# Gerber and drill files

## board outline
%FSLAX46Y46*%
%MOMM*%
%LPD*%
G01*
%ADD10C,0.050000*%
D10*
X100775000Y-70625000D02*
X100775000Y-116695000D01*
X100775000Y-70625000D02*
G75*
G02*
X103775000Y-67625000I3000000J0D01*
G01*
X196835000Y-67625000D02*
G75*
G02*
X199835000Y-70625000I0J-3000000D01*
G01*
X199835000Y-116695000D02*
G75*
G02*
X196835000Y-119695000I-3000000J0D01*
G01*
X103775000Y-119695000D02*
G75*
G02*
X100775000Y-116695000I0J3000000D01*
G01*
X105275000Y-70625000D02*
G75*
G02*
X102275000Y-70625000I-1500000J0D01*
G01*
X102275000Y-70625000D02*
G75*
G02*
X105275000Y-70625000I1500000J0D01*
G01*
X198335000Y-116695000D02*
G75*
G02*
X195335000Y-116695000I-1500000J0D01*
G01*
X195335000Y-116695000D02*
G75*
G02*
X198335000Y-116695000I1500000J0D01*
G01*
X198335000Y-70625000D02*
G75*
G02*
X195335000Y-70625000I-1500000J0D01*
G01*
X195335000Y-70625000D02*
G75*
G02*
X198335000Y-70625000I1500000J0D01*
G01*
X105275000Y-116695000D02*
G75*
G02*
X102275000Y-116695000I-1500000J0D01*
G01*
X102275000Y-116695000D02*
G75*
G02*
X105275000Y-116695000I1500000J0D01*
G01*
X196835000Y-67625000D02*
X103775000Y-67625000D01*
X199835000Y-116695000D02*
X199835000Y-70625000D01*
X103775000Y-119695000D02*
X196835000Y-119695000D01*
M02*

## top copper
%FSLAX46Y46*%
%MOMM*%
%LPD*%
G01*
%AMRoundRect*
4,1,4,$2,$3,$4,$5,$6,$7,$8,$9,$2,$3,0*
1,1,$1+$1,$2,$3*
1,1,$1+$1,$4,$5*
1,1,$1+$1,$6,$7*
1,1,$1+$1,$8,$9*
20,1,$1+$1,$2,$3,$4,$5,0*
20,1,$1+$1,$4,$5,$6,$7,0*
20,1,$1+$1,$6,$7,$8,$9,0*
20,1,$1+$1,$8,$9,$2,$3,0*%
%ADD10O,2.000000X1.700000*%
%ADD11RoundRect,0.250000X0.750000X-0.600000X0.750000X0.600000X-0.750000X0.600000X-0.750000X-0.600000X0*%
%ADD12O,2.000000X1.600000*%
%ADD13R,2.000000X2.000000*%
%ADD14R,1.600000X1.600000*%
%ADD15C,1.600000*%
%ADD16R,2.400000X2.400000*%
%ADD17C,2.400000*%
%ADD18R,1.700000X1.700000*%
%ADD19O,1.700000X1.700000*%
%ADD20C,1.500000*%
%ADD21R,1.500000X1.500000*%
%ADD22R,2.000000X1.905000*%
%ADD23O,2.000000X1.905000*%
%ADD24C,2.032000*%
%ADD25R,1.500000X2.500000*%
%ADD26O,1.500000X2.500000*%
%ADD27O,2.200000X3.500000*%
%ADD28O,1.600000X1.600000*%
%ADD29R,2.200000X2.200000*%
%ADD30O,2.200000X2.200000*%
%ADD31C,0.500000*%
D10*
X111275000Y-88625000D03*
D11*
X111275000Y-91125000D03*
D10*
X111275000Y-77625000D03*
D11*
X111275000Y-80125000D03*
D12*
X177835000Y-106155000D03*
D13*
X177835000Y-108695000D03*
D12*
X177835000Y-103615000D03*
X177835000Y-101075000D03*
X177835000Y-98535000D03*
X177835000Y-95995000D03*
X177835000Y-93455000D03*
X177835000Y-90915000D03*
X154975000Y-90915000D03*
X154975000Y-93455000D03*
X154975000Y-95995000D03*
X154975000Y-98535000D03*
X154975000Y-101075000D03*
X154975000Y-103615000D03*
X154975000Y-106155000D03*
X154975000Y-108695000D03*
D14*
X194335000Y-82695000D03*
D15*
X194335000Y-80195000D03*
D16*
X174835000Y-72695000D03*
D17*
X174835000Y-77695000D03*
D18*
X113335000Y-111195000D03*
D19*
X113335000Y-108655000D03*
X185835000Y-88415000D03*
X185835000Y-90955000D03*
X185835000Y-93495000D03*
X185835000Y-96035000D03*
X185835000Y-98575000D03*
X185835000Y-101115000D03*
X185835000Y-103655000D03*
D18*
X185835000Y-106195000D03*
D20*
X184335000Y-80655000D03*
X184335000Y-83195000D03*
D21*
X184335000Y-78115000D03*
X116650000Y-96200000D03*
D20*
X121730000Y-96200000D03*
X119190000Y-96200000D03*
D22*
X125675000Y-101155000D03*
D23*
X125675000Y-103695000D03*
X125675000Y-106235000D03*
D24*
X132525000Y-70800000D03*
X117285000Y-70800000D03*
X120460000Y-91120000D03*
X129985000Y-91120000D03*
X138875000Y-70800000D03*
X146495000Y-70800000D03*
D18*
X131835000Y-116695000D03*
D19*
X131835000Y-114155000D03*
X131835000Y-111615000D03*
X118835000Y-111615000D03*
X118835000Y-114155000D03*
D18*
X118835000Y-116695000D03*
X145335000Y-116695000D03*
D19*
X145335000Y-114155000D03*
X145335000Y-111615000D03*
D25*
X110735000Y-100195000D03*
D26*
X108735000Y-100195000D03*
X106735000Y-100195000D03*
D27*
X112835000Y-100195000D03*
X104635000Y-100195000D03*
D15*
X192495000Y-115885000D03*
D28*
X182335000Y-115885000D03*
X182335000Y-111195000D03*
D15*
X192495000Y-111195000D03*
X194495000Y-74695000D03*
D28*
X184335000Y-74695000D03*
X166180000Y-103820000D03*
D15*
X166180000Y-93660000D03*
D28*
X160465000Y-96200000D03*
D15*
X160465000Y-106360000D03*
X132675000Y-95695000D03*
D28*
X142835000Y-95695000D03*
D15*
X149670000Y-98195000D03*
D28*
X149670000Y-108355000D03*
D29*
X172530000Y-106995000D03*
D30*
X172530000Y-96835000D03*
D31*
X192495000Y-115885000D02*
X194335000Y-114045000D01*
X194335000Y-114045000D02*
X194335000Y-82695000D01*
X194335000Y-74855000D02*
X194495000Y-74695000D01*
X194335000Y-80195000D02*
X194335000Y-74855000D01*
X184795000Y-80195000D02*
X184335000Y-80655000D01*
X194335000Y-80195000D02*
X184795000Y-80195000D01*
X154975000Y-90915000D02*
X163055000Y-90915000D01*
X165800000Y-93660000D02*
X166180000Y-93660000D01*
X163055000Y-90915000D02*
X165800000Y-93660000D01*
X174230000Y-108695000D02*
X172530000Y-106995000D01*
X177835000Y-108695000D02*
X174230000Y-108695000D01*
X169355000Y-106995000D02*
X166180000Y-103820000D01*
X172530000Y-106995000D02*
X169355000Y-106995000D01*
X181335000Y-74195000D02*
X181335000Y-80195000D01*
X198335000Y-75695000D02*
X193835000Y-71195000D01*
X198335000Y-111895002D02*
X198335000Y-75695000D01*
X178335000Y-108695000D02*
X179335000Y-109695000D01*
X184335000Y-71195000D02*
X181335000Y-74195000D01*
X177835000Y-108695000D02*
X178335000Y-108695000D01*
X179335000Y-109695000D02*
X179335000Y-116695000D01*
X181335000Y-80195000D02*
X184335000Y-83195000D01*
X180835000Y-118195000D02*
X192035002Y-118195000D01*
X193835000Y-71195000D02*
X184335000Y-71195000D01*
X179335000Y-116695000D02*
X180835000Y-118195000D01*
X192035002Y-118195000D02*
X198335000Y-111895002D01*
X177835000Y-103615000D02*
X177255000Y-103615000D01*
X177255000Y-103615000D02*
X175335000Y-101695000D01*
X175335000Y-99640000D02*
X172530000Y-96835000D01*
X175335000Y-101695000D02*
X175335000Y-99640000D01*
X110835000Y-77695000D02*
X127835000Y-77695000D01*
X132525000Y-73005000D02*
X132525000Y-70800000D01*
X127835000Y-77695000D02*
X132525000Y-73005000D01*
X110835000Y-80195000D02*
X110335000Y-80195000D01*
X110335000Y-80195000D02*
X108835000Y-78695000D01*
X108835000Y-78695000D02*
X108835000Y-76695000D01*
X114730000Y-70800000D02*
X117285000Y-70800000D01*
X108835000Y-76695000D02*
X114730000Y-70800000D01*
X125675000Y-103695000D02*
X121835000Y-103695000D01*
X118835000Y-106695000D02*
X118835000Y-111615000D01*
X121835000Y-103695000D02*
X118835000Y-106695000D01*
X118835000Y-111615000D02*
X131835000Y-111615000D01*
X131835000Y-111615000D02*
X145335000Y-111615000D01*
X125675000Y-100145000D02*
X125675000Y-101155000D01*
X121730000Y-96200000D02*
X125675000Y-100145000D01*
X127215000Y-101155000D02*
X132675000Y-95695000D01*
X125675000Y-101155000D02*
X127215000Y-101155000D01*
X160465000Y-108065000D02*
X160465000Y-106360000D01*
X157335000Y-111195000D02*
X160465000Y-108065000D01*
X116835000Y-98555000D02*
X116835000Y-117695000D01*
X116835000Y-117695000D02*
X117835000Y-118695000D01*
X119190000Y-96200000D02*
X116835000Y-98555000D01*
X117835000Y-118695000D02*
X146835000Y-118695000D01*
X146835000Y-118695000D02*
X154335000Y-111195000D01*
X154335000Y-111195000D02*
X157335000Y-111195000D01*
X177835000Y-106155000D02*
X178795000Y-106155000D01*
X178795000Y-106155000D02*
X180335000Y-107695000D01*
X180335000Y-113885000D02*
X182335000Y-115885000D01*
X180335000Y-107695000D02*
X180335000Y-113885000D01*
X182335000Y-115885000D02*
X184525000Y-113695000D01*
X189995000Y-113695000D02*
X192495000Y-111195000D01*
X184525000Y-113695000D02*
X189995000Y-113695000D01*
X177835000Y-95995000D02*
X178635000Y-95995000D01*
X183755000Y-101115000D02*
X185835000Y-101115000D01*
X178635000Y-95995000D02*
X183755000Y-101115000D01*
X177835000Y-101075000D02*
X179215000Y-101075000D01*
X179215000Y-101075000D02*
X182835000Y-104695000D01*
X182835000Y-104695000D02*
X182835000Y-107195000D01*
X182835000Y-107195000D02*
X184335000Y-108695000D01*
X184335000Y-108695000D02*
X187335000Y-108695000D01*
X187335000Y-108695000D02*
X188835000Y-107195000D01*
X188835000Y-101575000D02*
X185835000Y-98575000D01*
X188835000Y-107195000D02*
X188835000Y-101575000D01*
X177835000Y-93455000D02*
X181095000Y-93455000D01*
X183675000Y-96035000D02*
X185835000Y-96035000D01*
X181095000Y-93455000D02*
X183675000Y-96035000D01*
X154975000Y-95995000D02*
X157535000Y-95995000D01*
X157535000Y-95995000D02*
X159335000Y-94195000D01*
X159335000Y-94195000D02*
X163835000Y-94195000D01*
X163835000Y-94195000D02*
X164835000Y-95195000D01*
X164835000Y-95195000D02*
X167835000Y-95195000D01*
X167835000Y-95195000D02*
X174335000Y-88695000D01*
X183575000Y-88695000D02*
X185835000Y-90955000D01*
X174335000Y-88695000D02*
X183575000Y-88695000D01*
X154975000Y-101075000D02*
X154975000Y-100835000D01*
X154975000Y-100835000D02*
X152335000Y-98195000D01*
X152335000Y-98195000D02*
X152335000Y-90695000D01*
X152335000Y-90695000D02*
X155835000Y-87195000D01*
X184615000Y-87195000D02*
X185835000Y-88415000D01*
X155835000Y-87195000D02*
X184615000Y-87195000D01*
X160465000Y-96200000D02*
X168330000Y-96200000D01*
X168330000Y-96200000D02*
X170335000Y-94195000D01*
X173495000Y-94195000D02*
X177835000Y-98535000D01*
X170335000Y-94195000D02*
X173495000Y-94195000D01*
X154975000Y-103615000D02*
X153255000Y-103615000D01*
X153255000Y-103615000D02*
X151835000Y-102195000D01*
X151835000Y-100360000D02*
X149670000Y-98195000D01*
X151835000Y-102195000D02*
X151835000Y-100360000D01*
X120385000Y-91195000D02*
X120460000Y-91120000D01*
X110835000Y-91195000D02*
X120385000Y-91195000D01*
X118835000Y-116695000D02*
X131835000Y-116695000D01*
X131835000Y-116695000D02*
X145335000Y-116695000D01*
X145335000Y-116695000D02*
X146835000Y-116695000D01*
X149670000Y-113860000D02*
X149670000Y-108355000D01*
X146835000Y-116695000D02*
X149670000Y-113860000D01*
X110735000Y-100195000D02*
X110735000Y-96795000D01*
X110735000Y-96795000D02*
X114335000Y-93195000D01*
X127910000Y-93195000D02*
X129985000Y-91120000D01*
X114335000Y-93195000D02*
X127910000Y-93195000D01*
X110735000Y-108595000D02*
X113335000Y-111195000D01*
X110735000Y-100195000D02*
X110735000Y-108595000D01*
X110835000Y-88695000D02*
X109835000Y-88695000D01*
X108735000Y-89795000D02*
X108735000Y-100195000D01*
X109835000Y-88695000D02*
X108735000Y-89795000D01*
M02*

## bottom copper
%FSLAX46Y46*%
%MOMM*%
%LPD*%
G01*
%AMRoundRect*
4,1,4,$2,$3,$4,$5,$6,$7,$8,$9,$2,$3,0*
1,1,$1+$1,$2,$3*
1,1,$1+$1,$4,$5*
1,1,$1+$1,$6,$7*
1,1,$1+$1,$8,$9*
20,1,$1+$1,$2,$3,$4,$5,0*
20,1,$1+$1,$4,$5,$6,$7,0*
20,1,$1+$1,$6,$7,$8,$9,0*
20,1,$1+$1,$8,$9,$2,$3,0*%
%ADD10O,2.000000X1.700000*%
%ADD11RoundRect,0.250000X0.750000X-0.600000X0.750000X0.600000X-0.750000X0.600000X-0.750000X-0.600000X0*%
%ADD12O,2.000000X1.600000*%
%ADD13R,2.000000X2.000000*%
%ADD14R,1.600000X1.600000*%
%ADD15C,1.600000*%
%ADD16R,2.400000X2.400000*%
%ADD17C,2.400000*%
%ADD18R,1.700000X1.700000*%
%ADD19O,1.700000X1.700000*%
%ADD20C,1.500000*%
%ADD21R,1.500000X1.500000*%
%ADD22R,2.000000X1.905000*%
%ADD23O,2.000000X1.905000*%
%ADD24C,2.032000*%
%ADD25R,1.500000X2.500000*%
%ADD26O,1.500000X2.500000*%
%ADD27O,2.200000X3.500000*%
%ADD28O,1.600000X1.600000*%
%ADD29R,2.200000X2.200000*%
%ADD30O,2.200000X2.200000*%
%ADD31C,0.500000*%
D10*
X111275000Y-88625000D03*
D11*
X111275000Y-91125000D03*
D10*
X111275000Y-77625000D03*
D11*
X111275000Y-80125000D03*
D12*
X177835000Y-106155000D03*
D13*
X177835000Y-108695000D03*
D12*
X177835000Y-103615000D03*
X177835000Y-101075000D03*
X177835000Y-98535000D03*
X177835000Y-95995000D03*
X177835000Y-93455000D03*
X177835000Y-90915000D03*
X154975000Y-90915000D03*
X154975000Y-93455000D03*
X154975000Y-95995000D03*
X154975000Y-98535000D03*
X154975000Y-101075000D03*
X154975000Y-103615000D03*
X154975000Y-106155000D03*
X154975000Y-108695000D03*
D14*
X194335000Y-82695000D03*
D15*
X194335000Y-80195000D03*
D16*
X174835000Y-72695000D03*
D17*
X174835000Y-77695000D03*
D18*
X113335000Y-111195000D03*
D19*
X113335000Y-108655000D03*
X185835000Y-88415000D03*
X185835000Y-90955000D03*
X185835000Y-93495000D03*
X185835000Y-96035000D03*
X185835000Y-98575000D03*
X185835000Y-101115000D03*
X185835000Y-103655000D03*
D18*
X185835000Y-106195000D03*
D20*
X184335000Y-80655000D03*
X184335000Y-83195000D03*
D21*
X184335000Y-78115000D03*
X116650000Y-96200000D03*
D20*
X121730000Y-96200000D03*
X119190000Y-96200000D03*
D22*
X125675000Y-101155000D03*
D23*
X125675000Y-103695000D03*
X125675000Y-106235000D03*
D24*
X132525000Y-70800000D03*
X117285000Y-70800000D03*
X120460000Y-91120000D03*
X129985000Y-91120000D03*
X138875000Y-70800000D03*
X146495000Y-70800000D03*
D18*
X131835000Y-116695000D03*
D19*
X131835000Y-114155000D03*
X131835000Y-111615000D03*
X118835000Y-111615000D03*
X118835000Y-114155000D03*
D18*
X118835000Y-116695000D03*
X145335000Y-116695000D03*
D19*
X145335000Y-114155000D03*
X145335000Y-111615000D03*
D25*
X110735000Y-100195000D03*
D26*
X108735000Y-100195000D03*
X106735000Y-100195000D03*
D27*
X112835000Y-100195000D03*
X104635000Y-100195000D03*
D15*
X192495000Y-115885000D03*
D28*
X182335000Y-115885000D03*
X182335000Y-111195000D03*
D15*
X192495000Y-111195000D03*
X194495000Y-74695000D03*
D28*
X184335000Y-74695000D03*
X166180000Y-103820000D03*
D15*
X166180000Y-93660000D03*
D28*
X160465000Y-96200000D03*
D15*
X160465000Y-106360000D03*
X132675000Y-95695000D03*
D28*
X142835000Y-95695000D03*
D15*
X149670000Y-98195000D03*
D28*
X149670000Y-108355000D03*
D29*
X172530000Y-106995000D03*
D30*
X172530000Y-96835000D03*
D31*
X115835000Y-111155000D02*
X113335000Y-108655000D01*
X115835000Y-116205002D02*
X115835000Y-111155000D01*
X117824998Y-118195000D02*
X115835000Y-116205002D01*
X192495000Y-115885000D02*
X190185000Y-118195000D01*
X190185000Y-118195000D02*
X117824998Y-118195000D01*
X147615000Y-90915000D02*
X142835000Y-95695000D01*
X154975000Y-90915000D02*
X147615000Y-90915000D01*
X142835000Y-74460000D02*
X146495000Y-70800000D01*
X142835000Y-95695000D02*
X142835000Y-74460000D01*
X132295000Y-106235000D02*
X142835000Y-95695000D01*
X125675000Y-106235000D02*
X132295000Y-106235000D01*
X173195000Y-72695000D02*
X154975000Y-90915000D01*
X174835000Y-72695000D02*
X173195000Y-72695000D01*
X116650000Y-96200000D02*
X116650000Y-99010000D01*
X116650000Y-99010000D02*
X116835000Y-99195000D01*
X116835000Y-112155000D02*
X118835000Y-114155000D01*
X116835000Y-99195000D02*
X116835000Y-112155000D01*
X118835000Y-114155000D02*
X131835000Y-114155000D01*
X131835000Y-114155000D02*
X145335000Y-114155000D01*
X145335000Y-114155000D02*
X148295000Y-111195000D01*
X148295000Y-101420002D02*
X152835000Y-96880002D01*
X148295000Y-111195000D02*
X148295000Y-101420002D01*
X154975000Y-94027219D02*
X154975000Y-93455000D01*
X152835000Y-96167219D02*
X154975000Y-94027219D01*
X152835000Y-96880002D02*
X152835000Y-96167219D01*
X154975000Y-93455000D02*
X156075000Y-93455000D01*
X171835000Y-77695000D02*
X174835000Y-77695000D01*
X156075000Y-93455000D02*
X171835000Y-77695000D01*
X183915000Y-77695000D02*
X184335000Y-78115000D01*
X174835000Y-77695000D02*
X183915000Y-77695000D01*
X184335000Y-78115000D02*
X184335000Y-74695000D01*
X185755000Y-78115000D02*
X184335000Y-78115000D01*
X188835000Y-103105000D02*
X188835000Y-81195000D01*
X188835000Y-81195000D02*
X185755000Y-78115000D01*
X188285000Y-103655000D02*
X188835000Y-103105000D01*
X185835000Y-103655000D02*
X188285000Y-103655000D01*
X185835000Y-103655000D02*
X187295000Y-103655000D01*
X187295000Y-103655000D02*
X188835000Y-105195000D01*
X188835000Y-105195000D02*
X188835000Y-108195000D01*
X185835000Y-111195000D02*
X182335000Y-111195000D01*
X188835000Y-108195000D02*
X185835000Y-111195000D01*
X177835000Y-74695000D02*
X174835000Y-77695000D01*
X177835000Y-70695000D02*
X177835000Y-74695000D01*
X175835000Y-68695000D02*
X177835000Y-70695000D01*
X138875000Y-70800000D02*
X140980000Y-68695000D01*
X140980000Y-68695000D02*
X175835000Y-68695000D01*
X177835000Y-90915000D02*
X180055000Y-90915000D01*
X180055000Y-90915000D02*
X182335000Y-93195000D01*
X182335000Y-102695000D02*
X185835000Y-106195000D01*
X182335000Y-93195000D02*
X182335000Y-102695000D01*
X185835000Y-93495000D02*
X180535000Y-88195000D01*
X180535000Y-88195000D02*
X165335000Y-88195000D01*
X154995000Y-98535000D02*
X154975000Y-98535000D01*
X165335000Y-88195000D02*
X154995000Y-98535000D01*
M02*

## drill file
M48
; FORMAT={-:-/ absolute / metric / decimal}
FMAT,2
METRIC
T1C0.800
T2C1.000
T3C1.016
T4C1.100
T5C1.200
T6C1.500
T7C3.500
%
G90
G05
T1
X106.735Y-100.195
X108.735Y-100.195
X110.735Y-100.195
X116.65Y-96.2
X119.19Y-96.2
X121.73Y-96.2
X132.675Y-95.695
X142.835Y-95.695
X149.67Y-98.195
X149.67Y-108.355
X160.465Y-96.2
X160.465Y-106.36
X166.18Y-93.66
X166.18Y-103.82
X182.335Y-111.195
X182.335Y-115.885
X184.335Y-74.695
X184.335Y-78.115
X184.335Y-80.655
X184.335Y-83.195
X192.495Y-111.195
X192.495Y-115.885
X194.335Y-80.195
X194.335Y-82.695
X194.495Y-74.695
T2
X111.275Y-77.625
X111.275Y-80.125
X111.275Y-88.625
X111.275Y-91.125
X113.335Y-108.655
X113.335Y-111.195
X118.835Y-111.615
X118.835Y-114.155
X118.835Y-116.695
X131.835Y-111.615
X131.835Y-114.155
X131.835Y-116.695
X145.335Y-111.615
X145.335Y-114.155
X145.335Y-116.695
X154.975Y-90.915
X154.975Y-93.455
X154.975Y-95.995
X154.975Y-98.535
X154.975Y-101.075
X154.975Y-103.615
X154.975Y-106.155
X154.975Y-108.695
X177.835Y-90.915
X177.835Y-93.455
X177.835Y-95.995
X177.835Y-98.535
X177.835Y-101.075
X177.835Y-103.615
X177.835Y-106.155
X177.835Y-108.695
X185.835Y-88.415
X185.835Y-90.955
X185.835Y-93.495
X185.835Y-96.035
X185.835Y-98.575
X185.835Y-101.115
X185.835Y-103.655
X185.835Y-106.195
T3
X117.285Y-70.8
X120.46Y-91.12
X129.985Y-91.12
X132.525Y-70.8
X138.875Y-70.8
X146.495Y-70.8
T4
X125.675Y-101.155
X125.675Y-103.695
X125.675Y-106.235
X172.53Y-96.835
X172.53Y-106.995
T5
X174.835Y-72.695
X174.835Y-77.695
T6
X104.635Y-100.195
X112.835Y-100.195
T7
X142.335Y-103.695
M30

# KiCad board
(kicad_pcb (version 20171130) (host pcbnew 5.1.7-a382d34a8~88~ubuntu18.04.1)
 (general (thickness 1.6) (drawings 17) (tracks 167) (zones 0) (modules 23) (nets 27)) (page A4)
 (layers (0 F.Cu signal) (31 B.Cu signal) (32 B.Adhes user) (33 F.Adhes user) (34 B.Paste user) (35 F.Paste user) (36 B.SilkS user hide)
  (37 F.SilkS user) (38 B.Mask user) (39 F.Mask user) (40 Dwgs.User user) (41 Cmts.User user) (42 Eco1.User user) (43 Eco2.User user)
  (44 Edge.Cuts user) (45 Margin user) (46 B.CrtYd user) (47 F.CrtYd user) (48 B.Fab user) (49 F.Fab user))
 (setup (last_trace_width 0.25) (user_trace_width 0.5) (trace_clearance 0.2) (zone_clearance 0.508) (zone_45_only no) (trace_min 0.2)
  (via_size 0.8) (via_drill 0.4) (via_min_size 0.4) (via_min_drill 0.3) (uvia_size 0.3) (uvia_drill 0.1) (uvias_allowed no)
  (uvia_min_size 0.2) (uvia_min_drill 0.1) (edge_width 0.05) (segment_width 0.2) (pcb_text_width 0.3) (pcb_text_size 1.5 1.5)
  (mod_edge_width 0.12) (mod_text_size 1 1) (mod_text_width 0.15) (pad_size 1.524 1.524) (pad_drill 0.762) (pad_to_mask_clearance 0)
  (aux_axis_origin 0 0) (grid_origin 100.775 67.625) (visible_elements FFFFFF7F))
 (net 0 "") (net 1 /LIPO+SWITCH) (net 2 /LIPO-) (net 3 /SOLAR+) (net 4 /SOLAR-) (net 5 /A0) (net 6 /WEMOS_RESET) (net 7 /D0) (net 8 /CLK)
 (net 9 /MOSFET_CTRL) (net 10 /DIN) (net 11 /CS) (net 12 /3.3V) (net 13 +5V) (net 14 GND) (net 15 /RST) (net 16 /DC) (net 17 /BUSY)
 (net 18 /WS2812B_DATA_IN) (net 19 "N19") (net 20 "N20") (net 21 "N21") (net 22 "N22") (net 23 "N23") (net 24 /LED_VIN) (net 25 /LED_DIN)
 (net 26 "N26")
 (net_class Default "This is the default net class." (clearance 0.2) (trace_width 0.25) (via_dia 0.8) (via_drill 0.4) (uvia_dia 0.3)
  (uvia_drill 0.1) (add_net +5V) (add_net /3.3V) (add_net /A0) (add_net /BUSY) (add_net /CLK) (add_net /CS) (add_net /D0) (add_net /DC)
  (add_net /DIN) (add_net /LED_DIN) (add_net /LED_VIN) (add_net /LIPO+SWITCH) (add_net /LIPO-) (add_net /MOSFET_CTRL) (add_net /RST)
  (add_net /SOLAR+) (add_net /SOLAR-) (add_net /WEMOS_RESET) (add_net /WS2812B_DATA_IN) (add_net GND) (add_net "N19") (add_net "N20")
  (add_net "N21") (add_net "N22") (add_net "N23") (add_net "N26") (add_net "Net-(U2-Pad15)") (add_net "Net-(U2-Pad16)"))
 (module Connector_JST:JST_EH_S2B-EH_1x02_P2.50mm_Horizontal (layer F.Cu) (at 111.275 91.125 90)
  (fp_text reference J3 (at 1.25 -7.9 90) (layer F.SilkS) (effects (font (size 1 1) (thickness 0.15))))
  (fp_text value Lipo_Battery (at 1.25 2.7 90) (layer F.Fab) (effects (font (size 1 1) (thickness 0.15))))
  (pad 2 thru_hole oval (at 2.5 0 90) (size 1.7 2) (drill 1) (layers *.Cu *.Mask) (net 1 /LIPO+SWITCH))
  (pad 1 thru_hole roundrect (at 0 0 90) (size 1.7 2) (drill 1) (layers *.Cu *.Mask) (roundrect_rratio 0.147059) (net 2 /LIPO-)))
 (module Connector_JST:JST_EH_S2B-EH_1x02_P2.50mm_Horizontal (layer F.Cu) (at 111.275 80.125 90)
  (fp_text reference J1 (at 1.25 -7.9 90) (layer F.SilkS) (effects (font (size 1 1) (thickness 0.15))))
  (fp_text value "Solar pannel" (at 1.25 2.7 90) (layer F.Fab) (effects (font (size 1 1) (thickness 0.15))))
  (pad 2 thru_hole oval (at 2.5 0 90) (size 1.7 2) (drill 1) (layers *.Cu *.Mask) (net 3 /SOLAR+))
  (pad 1 thru_hole roundrect (at 0 0 90) (size 1.7 2) (drill 1) (layers *.Cu *.Mask) (roundrect_rratio 0.147059) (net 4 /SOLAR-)))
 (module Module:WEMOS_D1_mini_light (layer F.Cu) (at 177.835 108.695 180)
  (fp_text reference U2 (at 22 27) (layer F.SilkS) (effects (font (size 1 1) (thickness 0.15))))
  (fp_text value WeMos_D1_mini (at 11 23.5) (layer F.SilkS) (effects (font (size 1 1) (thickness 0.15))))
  (pad 2 thru_hole oval (at 0 2.54 180) (size 2 1.6) (drill 1) (layers *.Cu *.Mask) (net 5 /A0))
  (pad 1 thru_hole rect (at 0 0 180) (size 2 2) (drill 1) (layers *.Cu *.Mask) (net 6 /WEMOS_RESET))
  (pad 3 thru_hole oval (at 0 5.08 180) (size 2 1.6) (drill 1) (layers *.Cu *.Mask) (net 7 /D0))
  (pad 4 thru_hole oval (at 0 7.62 180) (size 2 1.6) (drill 1) (layers *.Cu *.Mask) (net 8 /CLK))
  (pad 5 thru_hole oval (at 0 10.16 180) (size 2 1.6) (drill 1) (layers *.Cu *.Mask) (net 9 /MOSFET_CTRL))
  (pad 6 thru_hole oval (at 0 12.7 180) (size 2 1.6) (drill 1) (layers *.Cu *.Mask) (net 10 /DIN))
  (pad 7 thru_hole oval (at 0 15.24 180) (size 2 1.6) (drill 1) (layers *.Cu *.Mask) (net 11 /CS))
  (pad 8 thru_hole oval (at 0 17.78 180) (size 2 1.6) (drill 1) (layers *.Cu *.Mask) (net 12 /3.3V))
  (pad 9 thru_hole oval (at 22.86 17.78 180) (size 2 1.6) (drill 1) (layers *.Cu *.Mask) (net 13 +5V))
  (pad 10 thru_hole oval (at 22.86 15.24 180) (size 2 1.6) (drill 1) (layers *.Cu *.Mask) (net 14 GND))
  (pad 11 thru_hole oval (at 22.86 12.7 180) (size 2 1.6) (drill 1) (layers *.Cu *.Mask) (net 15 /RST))
  (pad 12 thru_hole oval (at 22.86 10.16 180) (size 2 1.6) (drill 1) (layers *.Cu *.Mask) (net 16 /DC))
  (pad 13 thru_hole oval (at 22.86 7.62 180) (size 2 1.6) (drill 1) (layers *.Cu *.Mask) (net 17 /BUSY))
  (pad 14 thru_hole oval (at 22.86 5.08 180) (size 2 1.6) (drill 1) (layers *.Cu *.Mask) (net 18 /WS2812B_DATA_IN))
  (pad 15 thru_hole oval (at 22.86 2.54 180) (size 2 1.6) (drill 1) (layers *.Cu *.Mask))
  (pad 16 thru_hole oval (at 22.86 0 180) (size 2 1.6) (drill 1) (layers *.Cu *.Mask)))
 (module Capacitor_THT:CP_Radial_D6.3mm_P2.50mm (layer F.Cu) (at 194.335 82.695 90)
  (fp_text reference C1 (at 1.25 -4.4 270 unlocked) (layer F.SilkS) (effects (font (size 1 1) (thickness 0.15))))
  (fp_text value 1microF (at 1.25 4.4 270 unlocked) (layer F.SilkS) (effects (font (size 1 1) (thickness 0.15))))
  (pad 1 thru_hole rect (at 0 0 90) (size 1.6 1.6) (drill 0.8) (layers *.Cu *.Mask) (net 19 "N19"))
  (pad 2 thru_hole circle (at 2.5 0 90) (size 1.6 1.6) (drill 0.8) (layers *.Cu *.Mask) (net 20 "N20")))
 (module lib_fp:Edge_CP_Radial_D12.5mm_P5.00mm (layer F.Cu) (at 174.835 75.195 270)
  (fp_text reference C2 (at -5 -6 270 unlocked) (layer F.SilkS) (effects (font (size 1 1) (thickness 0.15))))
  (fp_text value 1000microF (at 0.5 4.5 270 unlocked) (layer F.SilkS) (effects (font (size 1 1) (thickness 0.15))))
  (pad 1 thru_hole rect (at -2.5 0 270) (size 2.4 2.4) (drill 1.2) (layers *.Cu *.Mask) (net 13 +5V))
  (pad 2 thru_hole circle (at 2.5 0 270) (size 2.4 2.4) (drill 1.2) (layers *.Cu *.Mask) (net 14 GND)))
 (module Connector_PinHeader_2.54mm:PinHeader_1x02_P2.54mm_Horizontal (layer F.Cu) (at 113.335 111.195 180)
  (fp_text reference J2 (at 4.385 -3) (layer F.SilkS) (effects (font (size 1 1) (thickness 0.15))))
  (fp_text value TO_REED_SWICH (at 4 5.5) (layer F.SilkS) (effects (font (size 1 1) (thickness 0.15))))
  (pad 1 thru_hole rect (at 0 0 180) (size 1.7 1.7) (drill 1) (layers *.Cu *.Mask) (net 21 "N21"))
  (pad 2 thru_hole oval (at 0 2.54 180) (size 1.7 1.7) (drill 1) (layers *.Cu *.Mask) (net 19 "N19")))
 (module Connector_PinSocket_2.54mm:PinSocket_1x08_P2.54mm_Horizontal (layer F.Cu) (at 185.835 106.195 180)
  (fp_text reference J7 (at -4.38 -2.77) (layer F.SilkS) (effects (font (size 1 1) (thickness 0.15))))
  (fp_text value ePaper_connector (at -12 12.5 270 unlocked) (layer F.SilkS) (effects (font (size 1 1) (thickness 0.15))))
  (pad 8 thru_hole oval (at 0 17.78 180) (size 1.7 1.7) (drill 1) (layers *.Cu *.Mask) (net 17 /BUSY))
  (pad 7 thru_hole oval (at 0 15.24 180) (size 1.7 1.7) (drill 1) (layers *.Cu *.Mask) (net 15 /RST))
  (pad 6 thru_hole oval (at 0 12.7 180) (size 1.7 1.7) (drill 1) (layers *.Cu *.Mask) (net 16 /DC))
  (pad 5 thru_hole oval (at 0 10.16 180) (size 1.7 1.7) (drill 1) (layers *.Cu *.Mask) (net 11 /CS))
  (pad 4 thru_hole oval (at 0 7.62 180) (size 1.7 1.7) (drill 1) (layers *.Cu *.Mask) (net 8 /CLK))
  (pad 3 thru_hole oval (at 0 5.08 180) (size 1.7 1.7) (drill 1) (layers *.Cu *.Mask) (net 10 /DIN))
  (pad 2 thru_hole oval (at 0 2.54 180) (size 1.7 1.7) (drill 1) (layers *.Cu *.Mask) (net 14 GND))
  (pad 1 thru_hole rect (at 0 0 180) (size 1.7 1.7) (drill 1) (layers *.Cu *.Mask) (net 12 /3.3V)))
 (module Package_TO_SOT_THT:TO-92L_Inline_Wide (layer F.Cu) (at 184.335 78.115 270)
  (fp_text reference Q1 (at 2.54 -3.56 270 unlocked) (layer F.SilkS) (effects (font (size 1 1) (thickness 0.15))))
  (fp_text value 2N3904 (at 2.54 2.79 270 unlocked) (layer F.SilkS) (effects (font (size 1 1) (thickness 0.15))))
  (pad 2 thru_hole circle (at 2.54 0 270) (size 1.5 1.5) (drill 0.8) (layers *.Cu *.Mask) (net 20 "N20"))
  (pad 3 thru_hole circle (at 5.08 0 270) (size 1.5 1.5) (drill 0.8) (layers *.Cu *.Mask) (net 14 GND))
  (pad 1 thru_hole rect (at 0 0 270) (size 1.5 1.5) (drill 0.8) (layers *.Cu *.Mask) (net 6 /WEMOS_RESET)))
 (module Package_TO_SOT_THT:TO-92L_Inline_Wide (layer F.Cu) (at 116.65 96.2)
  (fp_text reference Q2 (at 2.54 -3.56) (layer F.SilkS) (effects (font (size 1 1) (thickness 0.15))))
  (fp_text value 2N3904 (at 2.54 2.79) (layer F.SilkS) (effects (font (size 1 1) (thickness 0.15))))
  (pad 1 thru_hole rect (at 0 0) (size 1.5 1.5) (drill 0.8) (layers *.Cu *.Mask) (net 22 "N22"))
  (pad 3 thru_hole circle (at 5.08 0) (size 1.5 1.5) (drill 0.8) (layers *.Cu *.Mask) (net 14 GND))
  (pad 2 thru_hole circle (at 2.54 0) (size 1.5 1.5) (drill 0.8) (layers *.Cu *.Mask) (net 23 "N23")))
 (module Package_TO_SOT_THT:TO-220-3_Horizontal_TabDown (layer F.Cu) (at 125.675 101.155 270)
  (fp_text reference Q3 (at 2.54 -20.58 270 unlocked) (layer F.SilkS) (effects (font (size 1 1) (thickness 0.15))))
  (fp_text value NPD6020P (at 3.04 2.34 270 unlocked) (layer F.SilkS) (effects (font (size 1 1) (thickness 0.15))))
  (pad "" np_thru_hole oval (at 2.54 -16.66 270) (size 3.5 3.5) (drill 3.5) (layers *.Cu *.Mask))
  (pad 1 thru_hole rect (at 0 0 270) (size 1.905 2) (drill 1.1) (layers *.Cu *.Mask) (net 22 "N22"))
  (pad 2 thru_hole oval (at 2.54 0 270) (size 1.905 2) (drill 1.1) (layers *.Cu *.Mask) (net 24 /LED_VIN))
  (pad 3 thru_hole oval (at 5.08 0 270) (size 1.905 2) (drill 1.1) (layers *.Cu *.Mask) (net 13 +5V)))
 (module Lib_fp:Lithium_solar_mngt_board (layer F.Cu) (at 135.065 66.99)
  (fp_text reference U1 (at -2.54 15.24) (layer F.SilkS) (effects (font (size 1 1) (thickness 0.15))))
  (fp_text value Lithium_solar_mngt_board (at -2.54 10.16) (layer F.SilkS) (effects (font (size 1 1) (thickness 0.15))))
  (pad 1 thru_hole circle (at -2.54 3.81) (size 2.032 2.032) (drill 1.016) (layers *.Cu *.Mask) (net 3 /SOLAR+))
  (pad 2 thru_hole circle (at -17.78 3.81) (size 2.032 2.032) (drill 1.016) (layers *.Cu *.Mask) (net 4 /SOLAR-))
  (pad 4 thru_hole circle (at -14.605 24.13) (size 2.032 2.032) (drill 1.016) (layers *.Cu *.Mask) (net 2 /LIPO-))
  (pad 3 thru_hole circle (at -5.08 24.13) (size 2.032 2.032) (drill 1.016) (layers *.Cu *.Mask) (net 21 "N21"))
  (pad 6 thru_hole circle (at 3.81 3.81) (size 2.032 2.032) (drill 1.016) (layers *.Cu *.Mask) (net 14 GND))
  (pad 5 thru_hole circle (at 11.43 3.81) (size 2.032 2.032) (drill 1.016) (layers *.Cu *.Mask) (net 13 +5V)))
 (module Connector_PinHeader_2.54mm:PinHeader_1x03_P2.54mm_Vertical (layer F.Cu) (at 131.835 116.695 180)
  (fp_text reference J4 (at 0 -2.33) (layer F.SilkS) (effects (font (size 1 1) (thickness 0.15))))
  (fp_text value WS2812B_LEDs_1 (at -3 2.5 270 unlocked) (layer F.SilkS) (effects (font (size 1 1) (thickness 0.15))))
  (pad 1 thru_hole rect (at 0 0 180) (size 1.7 1.7) (drill 1) (layers *.Cu *.Mask) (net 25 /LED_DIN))
  (pad 2 thru_hole oval (at 0 2.54 180) (size 1.7 1.7) (drill 1) (layers *.Cu *.Mask) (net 14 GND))
  (pad 3 thru_hole oval (at 0 5.08 180) (size 1.7 1.7) (drill 1) (layers *.Cu *.Mask) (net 24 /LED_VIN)))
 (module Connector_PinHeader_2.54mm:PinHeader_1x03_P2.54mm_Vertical (layer F.Cu) (at 118.835 116.695 180)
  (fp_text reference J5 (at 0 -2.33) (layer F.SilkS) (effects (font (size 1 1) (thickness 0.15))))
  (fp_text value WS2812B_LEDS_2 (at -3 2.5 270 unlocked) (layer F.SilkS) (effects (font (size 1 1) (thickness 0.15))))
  (pad 3 thru_hole oval (at 0 5.08 180) (size 1.7 1.7) (drill 1) (layers *.Cu *.Mask) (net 24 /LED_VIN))
  (pad 2 thru_hole oval (at 0 2.54 180) (size 1.7 1.7) (drill 1) (layers *.Cu *.Mask) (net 14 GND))
  (pad 1 thru_hole rect (at 0 0 180) (size 1.7 1.7) (drill 1) (layers *.Cu *.Mask) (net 25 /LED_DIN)))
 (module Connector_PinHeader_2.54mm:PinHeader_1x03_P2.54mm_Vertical (layer F.Cu) (at 145.335 116.695 180)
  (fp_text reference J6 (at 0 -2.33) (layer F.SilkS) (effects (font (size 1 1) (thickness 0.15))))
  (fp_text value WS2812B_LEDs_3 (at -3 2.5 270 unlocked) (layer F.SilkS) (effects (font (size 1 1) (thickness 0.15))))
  (pad 1 thru_hole rect (at 0 0 180) (size 1.7 1.7) (drill 1) (layers *.Cu *.Mask) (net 25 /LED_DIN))
  (pad 2 thru_hole oval (at 0 2.54 180) (size 1.7 1.7) (drill 1) (layers *.Cu *.Mask) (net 14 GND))
  (pad 3 thru_hole oval (at 0 5.08 180) (size 1.7 1.7) (drill 1) (layers *.Cu *.Mask) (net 24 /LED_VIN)))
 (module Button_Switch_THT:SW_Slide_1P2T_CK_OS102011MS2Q (layer F.Cu) (at 110.735 100.195 180)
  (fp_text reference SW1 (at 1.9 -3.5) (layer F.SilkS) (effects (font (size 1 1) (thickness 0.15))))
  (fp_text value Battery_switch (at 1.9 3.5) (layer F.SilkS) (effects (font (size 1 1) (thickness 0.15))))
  (pad 1 thru_hole rect (at 0 0 180) (size 1.5 2.5) (drill 0.8) (layers *.Cu *.Mask) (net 21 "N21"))
  (pad 2 thru_hole oval (at 2 0 180) (size 1.5 2.5) (drill 0.8) (layers *.Cu *.Mask) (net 1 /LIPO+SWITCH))
  (pad 3 thru_hole oval (at 4 0 180) (size 1.5 2.5) (drill 0.8) (layers *.Cu *.Mask))
  (pad "" thru_hole oval (at -2.1 0 180) (size 2.2 3.5) (drill 1.5) (layers *.Cu *.Mask))
  (pad "" thru_hole oval (at 6.1 0 180) (size 2.2 3.5) (drill 1.5) (layers *.Cu *.Mask)))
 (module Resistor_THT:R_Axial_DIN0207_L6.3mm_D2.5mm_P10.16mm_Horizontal (layer F.Cu) (at 192.495 115.885 180)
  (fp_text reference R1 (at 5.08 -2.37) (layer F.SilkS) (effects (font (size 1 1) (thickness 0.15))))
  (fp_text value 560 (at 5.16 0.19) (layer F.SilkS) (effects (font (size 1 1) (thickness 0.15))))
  (pad 1 thru_hole circle (at 0 0 180) (size 1.6 1.6) (drill 0.8) (layers *.Cu *.Mask) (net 19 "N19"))
  (pad 2 thru_hole oval (at 10.16 0 180) (size 1.6 1.6) (drill 0.8) (layers *.Cu *.Mask) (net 5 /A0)))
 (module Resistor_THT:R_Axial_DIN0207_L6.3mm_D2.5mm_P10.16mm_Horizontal (layer F.Cu) (at 192.495 111.195 180)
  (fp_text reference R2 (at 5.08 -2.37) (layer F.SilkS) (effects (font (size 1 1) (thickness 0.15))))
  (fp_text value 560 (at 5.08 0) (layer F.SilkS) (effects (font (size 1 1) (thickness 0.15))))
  (pad 2 thru_hole oval (at 10.16 0 180) (size 1.6 1.6) (drill 0.8) (layers *.Cu *.Mask) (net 14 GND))
  (pad 1 thru_hole circle (at 0 0 180) (size 1.6 1.6) (drill 0.8) (layers *.Cu *.Mask) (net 5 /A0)))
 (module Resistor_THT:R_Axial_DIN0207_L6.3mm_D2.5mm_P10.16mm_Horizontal (layer F.Cu) (at 194.495 74.695 180)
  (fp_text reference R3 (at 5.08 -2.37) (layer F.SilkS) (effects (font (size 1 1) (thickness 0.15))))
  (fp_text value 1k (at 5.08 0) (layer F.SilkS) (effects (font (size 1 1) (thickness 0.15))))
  (pad 1 thru_hole circle (at 0 0 180) (size 1.6 1.6) (drill 0.8) (layers *.Cu *.Mask) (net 20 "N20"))
  (pad 2 thru_hole oval (at 10.16 0 180) (size 1.6 1.6) (drill 0.8) (layers *.Cu *.Mask) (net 14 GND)))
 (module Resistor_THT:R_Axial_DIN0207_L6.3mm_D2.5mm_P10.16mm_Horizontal (layer F.Cu) (at 166.18 93.66 270)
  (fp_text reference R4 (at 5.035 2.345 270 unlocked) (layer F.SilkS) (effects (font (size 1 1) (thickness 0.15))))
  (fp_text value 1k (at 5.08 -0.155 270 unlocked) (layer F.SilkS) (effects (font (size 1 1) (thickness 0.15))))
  (pad 2 thru_hole oval (at 10.16 0 270) (size 1.6 1.6) (drill 0.8) (layers *.Cu *.Mask) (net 6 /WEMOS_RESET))
  (pad 1 thru_hole circle (at 0 0 270) (size 1.6 1.6) (drill 0.8) (layers *.Cu *.Mask) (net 13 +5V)))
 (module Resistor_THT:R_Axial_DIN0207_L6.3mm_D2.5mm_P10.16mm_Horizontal (layer F.Cu) (at 160.465 106.36 90)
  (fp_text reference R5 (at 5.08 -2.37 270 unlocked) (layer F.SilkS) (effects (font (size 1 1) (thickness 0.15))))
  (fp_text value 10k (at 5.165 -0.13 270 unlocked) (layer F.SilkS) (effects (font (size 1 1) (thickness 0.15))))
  (pad 2 thru_hole oval (at 10.16 0 90) (size 1.6 1.6) (drill 0.8) (layers *.Cu *.Mask) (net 9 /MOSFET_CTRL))
  (pad 1 thru_hole circle (at 0 0 90) (size 1.6 1.6) (drill 0.8) (layers *.Cu *.Mask) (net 23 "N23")))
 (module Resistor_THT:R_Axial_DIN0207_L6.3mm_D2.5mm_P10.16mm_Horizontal (layer F.Cu) (at 132.675 95.695)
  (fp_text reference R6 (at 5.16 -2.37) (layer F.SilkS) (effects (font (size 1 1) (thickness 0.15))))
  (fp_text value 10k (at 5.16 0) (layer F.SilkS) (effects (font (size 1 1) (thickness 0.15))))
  (pad 1 thru_hole circle (at 0 0) (size 1.6 1.6) (drill 0.8) (layers *.Cu *.Mask) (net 22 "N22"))
  (pad 2 thru_hole oval (at 10.16 0) (size 1.6 1.6) (drill 0.8) (layers *.Cu *.Mask) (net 13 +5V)))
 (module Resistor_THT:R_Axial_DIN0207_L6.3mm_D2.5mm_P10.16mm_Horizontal (layer F.Cu) (at 149.67 98.195 270)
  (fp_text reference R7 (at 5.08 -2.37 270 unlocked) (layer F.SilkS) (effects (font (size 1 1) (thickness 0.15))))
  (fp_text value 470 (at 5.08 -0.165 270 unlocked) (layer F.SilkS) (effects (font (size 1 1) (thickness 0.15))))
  (pad 1 thru_hole circle (at 0 0 270) (size 1.6 1.6) (drill 0.8) (layers *.Cu *.Mask) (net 18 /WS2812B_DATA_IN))
  (pad 2 thru_hole oval (at 10.16 0 270) (size 1.6 1.6) (drill 0.8) (layers *.Cu *.Mask) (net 25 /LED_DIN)))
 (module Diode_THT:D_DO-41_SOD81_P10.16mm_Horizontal (layer F.Cu) (at 172.53 106.995 90)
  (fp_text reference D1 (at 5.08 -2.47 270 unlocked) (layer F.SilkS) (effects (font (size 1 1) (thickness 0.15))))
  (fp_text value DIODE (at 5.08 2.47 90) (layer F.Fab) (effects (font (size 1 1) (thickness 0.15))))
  (pad 1 thru_hole rect (at 0 0 90) (size 2.2 2.2) (drill 1.1) (layers *.Cu *.Mask) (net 6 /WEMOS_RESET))
  (pad 2 thru_hole oval (at 10.16 0 90) (size 2.2 2.2) (drill 1.1) (layers *.Cu *.Mask) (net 7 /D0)))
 (gr_line (start 100.775 70.625) (end 100.775 116.695) (layer Edge.Cuts) (width 0.05))
 (gr_arc (start 103.775 70.625) (end 103.775 67.625) (angle -90) (layer Edge.Cuts) (width 0.05))
 (gr_arc (start 196.835 70.625) (end 199.835 70.625) (angle -90) (layer Edge.Cuts) (width 0.05))
 (gr_arc (start 196.835 116.695) (end 196.835 119.695) (angle -90) (layer Edge.Cuts) (width 0.05))
 (gr_arc (start 103.775 116.695) (end 100.775 116.695) (angle -90) (layer Edge.Cuts) (width 0.05))
 (gr_circle (center 103.775 70.625) (end 102.275 70.625) (layer Edge.Cuts) (width 0.05))
 (gr_circle (center 196.835 116.695) (end 198.335 116.695) (layer Edge.Cuts) (width 0.05))
 (gr_circle (center 196.835 70.625) (end 198.335 70.625) (layer Edge.Cuts) (width 0.05))
 (gr_circle (center 103.775 116.695) (end 102.275 116.695) (layer Edge.Cuts) (width 0.05))
 (gr_line (start 196.835 67.625) (end 103.775 67.625) (layer Edge.Cuts) (width 0.05))
 (gr_line (start 199.835 116.695) (end 199.835 70.625) (layer Edge.Cuts) (width 0.05))
 (gr_line (start 103.775 119.695) (end 196.835 119.695) (layer Edge.Cuts) (width 0.05))
 (segment (start 192.495 115.885) (end 194.335 114.045) (width 0.5) (layer F.Cu) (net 19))
 (segment (start 194.335 114.045) (end 194.335 82.695) (width 0.5) (layer F.Cu) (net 19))
 (segment (start 115.835 111.155) (end 113.335 108.655) (width 0.5) (layer B.Cu) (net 19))
 (segment (start 115.835 116.205002) (end 115.835 111.155) (width 0.5) (layer B.Cu) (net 19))
 (segment (start 117.824998 118.195) (end 115.835 116.205002) (width 0.5) (layer B.Cu) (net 19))
 (segment (start 192.495 115.885) (end 190.185 118.195) (width 0.5) (layer B.Cu) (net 19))
 (segment (start 190.185 118.195) (end 117.824998 118.195) (width 0.5) (layer B.Cu) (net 19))
 (segment (start 194.335 74.855) (end 194.495 74.695) (width 0.5) (layer F.Cu) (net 20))
 (segment (start 194.335 80.195) (end 194.335 74.855) (width 0.5) (layer F.Cu) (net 20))
 (segment (start 184.795 80.195) (end 184.335 80.655) (width 0.5) (layer F.Cu) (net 20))
 (segment (start 194.335 80.195) (end 184.795 80.195) (width 0.5) (layer F.Cu) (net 20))
 (segment (start 154.975 90.915) (end 163.055 90.915) (width 0.5) (layer F.Cu) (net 13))
 (segment (start 165.8 93.66) (end 166.18 93.66) (width 0.5) (layer F.Cu) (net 13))
 (segment (start 163.055 90.915) (end 165.8 93.66) (width 0.5) (layer F.Cu) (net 13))
 (segment (start 147.615 90.915) (end 142.835 95.695) (width 0.5) (layer B.Cu) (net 13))
 (segment (start 154.975 90.915) (end 147.615 90.915) (width 0.5) (layer B.Cu) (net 13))
 (segment (start 142.835 74.46) (end 146.495 70.8) (width 0.5) (layer B.Cu) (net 13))
 (segment (start 142.835 95.695) (end 142.835 74.46) (width 0.5) (layer B.Cu) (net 13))
 (segment (start 132.295 106.235) (end 142.835 95.695) (width 0.5) (layer B.Cu) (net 13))
 (segment (start 125.675 106.235) (end 132.295 106.235) (width 0.5) (layer B.Cu) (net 13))
 (segment (start 173.195 72.695) (end 154.975 90.915) (width 0.5) (layer B.Cu) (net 13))
 (segment (start 174.835 72.695) (end 173.195 72.695) (width 0.5) (layer B.Cu) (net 13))
 (segment (start 116.65 96.2) (end 116.65 99.01) (width 0.5) (layer B.Cu) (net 14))
 (segment (start 116.65 99.01) (end 116.835 99.195) (width 0.5) (layer B.Cu) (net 14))
 (segment (start 116.835 112.155) (end 118.835 114.155) (width 0.5) (layer B.Cu) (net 14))
 (segment (start 116.835 99.195) (end 116.835 112.155) (width 0.5) (layer B.Cu) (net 14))
 (segment (start 118.835 114.155) (end 131.835 114.155) (width 0.5) (layer B.Cu) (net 14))
 (segment (start 131.835 114.155) (end 145.335 114.155) (width 0.5) (layer B.Cu) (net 14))
 (segment (start 145.335 114.155) (end 148.295 111.195) (width 0.5) (layer B.Cu) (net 14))
 (segment (start 148.295 101.420002) (end 152.835 96.880002) (width 0.5) (layer B.Cu) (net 14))
 (segment (start 148.295 111.195) (end 148.295 101.420002) (width 0.5) (layer B.Cu) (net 14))
 (segment (start 154.975 94.027219) (end 154.975 93.455) (width 0.5) (layer B.Cu) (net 14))
 (segment (start 152.835 96.167219) (end 154.975 94.027219) (width 0.5) (layer B.Cu) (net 14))
 (segment (start 152.835 96.880002) (end 152.835 96.167219) (width 0.5) (layer B.Cu) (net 14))
 (segment (start 154.975 93.455) (end 156.075 93.455) (width 0.5) (layer B.Cu) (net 14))
 (segment (start 171.835 77.695) (end 174.835 77.695) (width 0.5) (layer B.Cu) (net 14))
 (segment (start 156.075 93.455) (end 171.835 77.695) (width 0.5) (layer B.Cu) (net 14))
 (segment (start 183.915 77.695) (end 184.335 78.115) (width 0.5) (layer B.Cu) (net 14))
 (segment (start 174.835 77.695) (end 183.915 77.695) (width 0.5) (layer B.Cu) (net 14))
 (segment (start 184.335 78.115) (end 184.335 74.695) (width 0.5) (layer B.Cu) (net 14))
 (segment (start 185.755 78.115) (end 184.335 78.115) (width 0.5) (layer B.Cu) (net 14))
 (segment (start 188.835 103.105) (end 188.835 81.195) (width 0.5) (layer B.Cu) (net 14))
 (segment (start 188.835 81.195) (end 185.755 78.115) (width 0.5) (layer B.Cu) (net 14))
 (segment (start 188.285 103.655) (end 188.835 103.105) (width 0.5) (layer B.Cu) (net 14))
 (segment (start 185.835 103.655) (end 188.285 103.655) (width 0.5) (layer B.Cu) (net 14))
 (segment (start 185.835 103.655) (end 187.295 103.655) (width 0.5) (layer B.Cu) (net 14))
 (segment (start 187.295 103.655) (end 188.835 105.195) (width 0.5) (layer B.Cu) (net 14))
 (segment (start 188.835 105.195) (end 188.835 108.195) (width 0.5) (layer B.Cu) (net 14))
 (segment (start 185.835 111.195) (end 182.335 111.195) (width 0.5) (layer B.Cu) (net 14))
 (segment (start 188.835 108.195) (end 185.835 111.195) (width 0.5) (layer B.Cu) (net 14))
 (segment (start 177.835 74.695) (end 174.835 77.695) (width 0.5) (layer B.Cu) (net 14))
 (segment (start 177.835 70.695) (end 177.835 74.695) (width 0.5) (layer B.Cu) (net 14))
 (segment (start 175.835 68.695) (end 177.835 70.695) (width 0.5) (layer B.Cu) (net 14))
 (segment (start 138.875 70.8) (end 140.98 68.695) (width 0.5) (layer B.Cu) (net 14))
 (segment (start 140.98 68.695) (end 175.835 68.695) (width 0.5) (layer B.Cu) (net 14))
 (segment (start 174.23 108.695) (end 172.53 106.995) (width 0.5) (layer F.Cu) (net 6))
 (segment (start 177.835 108.695) (end 174.23 108.695) (width 0.5) (layer F.Cu) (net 6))
 (segment (start 169.355 106.995) (end 166.18 103.82) (width 0.5) (layer F.Cu) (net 6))
 (segment (start 172.53 106.995) (end 169.355 106.995) (width 0.5) (layer F.Cu) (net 6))
 (segment (start 181.335 74.195) (end 181.335 80.195) (width 0.5) (layer F.Cu) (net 6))
 (segment (start 198.335 75.695) (end 193.835 71.195) (width 0.5) (layer F.Cu) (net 6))
 (segment (start 198.335 111.895002) (end 198.335 75.695) (width 0.5) (layer F.Cu) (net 6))
 (segment (start 178.335 108.695) (end 179.335 109.695) (width 0.5) (layer F.Cu) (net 6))
 (segment (start 184.335 71.195) (end 181.335 74.195) (width 0.5) (layer F.Cu) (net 6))
 (segment (start 177.835 108.695) (end 178.335 108.695) (width 0.5) (layer F.Cu) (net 6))
 (segment (start 179.335 109.695) (end 179.335 116.695) (width 0.5) (layer F.Cu) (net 6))
 (segment (start 181.335 80.195) (end 184.335 83.195) (width 0.5) (layer F.Cu) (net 6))
 (segment (start 180.835 118.195) (end 192.035002 118.195) (width 0.5) (layer F.Cu) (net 6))
 (segment (start 193.835 71.195) (end 184.335 71.195) (width 0.5) (layer F.Cu) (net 6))
 (segment (start 179.335 116.695) (end 180.835 118.195) (width 0.5) (layer F.Cu) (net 6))
 (segment (start 192.035002 118.195) (end 198.335 111.895002) (width 0.5) (layer F.Cu) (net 6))
 (segment (start 177.835 103.615) (end 177.255 103.615) (width 0.5) (layer F.Cu) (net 7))
 (segment (start 177.255 103.615) (end 175.335 101.695) (width 0.5) (layer F.Cu) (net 7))
 (segment (start 175.335 99.64) (end 172.53 96.835) (width 0.5) (layer F.Cu) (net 7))
 (segment (start 175.335 101.695) (end 175.335 99.64) (width 0.5) (layer F.Cu) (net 7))
 (segment (start 110.835 77.695) (end 127.835 77.695) (width 0.5) (layer F.Cu) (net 3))
 (segment (start 132.525 73.005) (end 132.525 70.8) (width 0.5) (layer F.Cu) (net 3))
 (segment (start 127.835 77.695) (end 132.525 73.005) (width 0.5) (layer F.Cu) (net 3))
 (segment (start 110.835 80.195) (end 110.335 80.195) (width 0.5) (layer F.Cu) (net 4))
 (segment (start 110.335 80.195) (end 108.835 78.695) (width 0.5) (layer F.Cu) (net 4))
 (segment (start 108.835 78.695) (end 108.835 76.695) (width 0.5) (layer F.Cu) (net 4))
 (segment (start 114.73 70.8) (end 117.285 70.8) (width 0.5) (layer F.Cu) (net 4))
 (segment (start 108.835 76.695) (end 114.73 70.8) (width 0.5) (layer F.Cu) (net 4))
 (segment (start 125.675 103.695) (end 121.835 103.695) (width 0.5) (layer F.Cu) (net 24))
 (segment (start 118.835 106.695) (end 118.835 111.615) (width 0.5) (layer F.Cu) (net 24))
 (segment (start 121.835 103.695) (end 118.835 106.695) (width 0.5) (layer F.Cu) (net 24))
 (segment (start 118.835 111.615) (end 131.835 111.615) (width 0.5) (layer F.Cu) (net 24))
 (segment (start 131.835 111.615) (end 145.335 111.615) (width 0.5) (layer F.Cu) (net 24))
 (segment (start 177.835 90.915) (end 180.055 90.915) (width 0.5) (layer B.Cu) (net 12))
 (segment (start 180.055 90.915) (end 182.335 93.195) (width 0.5) (layer B.Cu) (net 12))
 (segment (start 182.335 102.695) (end 185.835 106.195) (width 0.5) (layer B.Cu) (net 12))
 (segment (start 182.335 93.195) (end 182.335 102.695) (width 0.5) (layer B.Cu) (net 12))
 (segment (start 125.675 100.145) (end 125.675 101.155) (width 0.5) (layer F.Cu) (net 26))
 (segment (start 121.73 96.2) (end 125.675 100.145) (width 0.5) (layer F.Cu) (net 26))
 (segment (start 127.215 101.155) (end 132.675 95.695) (width 0.5) (layer F.Cu) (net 26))
 (segment (start 125.675 101.155) (end 127.215 101.155) (width 0.5) (layer F.Cu) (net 26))
 (segment (start 160.465 108.065) (end 160.465 106.36) (width 0.5) (layer F.Cu) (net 23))
 (segment (start 157.335 111.195) (end 160.465 108.065) (width 0.5) (layer F.Cu) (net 23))
 (segment (start 116.835 98.555) (end 116.835 117.695) (width 0.5) (layer F.Cu) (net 23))
 (segment (start 116.835 117.695) (end 117.835 118.695) (width 0.5) (layer F.Cu) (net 23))
 (segment (start 119.19 96.2) (end 116.835 98.555) (width 0.5) (layer F.Cu) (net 23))
 (segment (start 117.835 118.695) (end 146.835 118.695) (width 0.5) (layer F.Cu) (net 23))
 (segment (start 146.835 118.695) (end 154.335 111.195) (width 0.5) (layer F.Cu) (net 23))
 (segment (start 154.335 111.195) (end 157.335 111.195) (width 0.5) (layer F.Cu) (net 23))
 (segment (start 177.835 106.155) (end 178.795 106.155) (width 0.5) (layer F.Cu) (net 5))
 (segment (start 178.795 106.155) (end 180.335 107.695) (width 0.5) (layer F.Cu) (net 5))
 (segment (start 180.335 113.885) (end 182.335 115.885) (width 0.5) (layer F.Cu) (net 5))
 (segment (start 180.335 107.695) (end 180.335 113.885) (width 0.5) (layer F.Cu) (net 5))
 (segment (start 182.335 115.885) (end 184.525 113.695) (width 0.5) (layer F.Cu) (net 5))
 (segment (start 189.995 113.695) (end 192.495 111.195) (width 0.5) (layer F.Cu) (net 5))
 (segment (start 184.525 113.695) (end 189.995 113.695) (width 0.5) (layer F.Cu) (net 5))
 (segment (start 177.835 95.995) (end 178.635 95.995) (width 0.5) (layer F.Cu) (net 10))
 (segment (start 183.755 101.115) (end 185.835 101.115) (width 0.5) (layer F.Cu) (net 10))
 (segment (start 178.635 95.995) (end 183.755 101.115) (width 0.5) (layer F.Cu) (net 10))
 (segment (start 177.835 101.075) (end 179.215 101.075) (width 0.5) (layer F.Cu) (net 8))
 (segment (start 179.215 101.075) (end 182.835 104.695) (width 0.5) (layer F.Cu) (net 8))
 (segment (start 182.835 104.695) (end 182.835 107.195) (width 0.5) (layer F.Cu) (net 8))
 (segment (start 182.835 107.195) (end 184.335 108.695) (width 0.5) (layer F.Cu) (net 8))
 (segment (start 184.335 108.695) (end 187.335 108.695) (width 0.5) (layer F.Cu) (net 8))
 (segment (start 187.335 108.695) (end 188.835 107.195) (width 0.5) (layer F.Cu) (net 8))
 (segment (start 188.835 101.575) (end 185.835 98.575) (width 0.5) (layer F.Cu) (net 8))
 (segment (start 188.835 107.195) (end 188.835 101.575) (width 0.5) (layer F.Cu) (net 8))
 (segment (start 177.835 93.455) (end 181.095 93.455) (width 0.5) (layer F.Cu) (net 11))
 (segment (start 183.675 96.035) (end 185.835 96.035) (width 0.5) (layer F.Cu) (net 11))
 (segment (start 181.095 93.455) (end 183.675 96.035) (width 0.5) (layer F.Cu) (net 11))
 (segment (start 185.835 93.495) (end 180.535 88.195) (width 0.5) (layer B.Cu) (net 16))
 (segment (start 180.535 88.195) (end 165.335 88.195) (width 0.5) (layer B.Cu) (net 16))
 (segment (start 154.995 98.535) (end 154.975 98.535) (width 0.5) (layer B.Cu) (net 16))
 (segment (start 165.335 88.195) (end 154.995 98.535) (width 0.5) (layer B.Cu) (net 16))
 (segment (start 154.975 95.995) (end 157.535 95.995) (width 0.5) (layer F.Cu) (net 15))
 (segment (start 157.535 95.995) (end 159.335 94.195) (width 0.5) (layer F.Cu) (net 15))
 (segment (start 159.335 94.195) (end 163.835 94.195) (width 0.5) (layer F.Cu) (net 15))
 (segment (start 163.835 94.195) (end 164.835 95.195) (width 0.5) (layer F.Cu) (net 15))
 (segment (start 164.835 95.195) (end 167.835 95.195) (width 0.5) (layer F.Cu) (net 15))
 (segment (start 167.835 95.195) (end 174.335 88.695) (width 0.5) (layer F.Cu) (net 15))
 (segment (start 183.575 88.695) (end 185.835 90.955) (width 0.5) (layer F.Cu) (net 15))
 (segment (start 174.335 88.695) (end 183.575 88.695) (width 0.5) (layer F.Cu) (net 15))
 (segment (start 154.975 101.075) (end 154.975 100.835) (width 0.5) (layer F.Cu) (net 17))
 (segment (start 154.975 100.835) (end 152.335 98.195) (width 0.5) (layer F.Cu) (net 17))
 (segment (start 152.335 98.195) (end 152.335 90.695) (width 0.5) (layer F.Cu) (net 17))
 (segment (start 152.335 90.695) (end 155.835 87.195) (width 0.5) (layer F.Cu) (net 17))
 (segment (start 184.615 87.195) (end 185.835 88.415) (width 0.5) (layer F.Cu) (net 17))
 (segment (start 155.835 87.195) (end 184.615 87.195) (width 0.5) (layer F.Cu) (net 17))
 (segment (start 160.465 96.2) (end 168.33 96.2) (width 0.5) (layer F.Cu) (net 9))
 (segment (start 168.33 96.2) (end 170.335 94.195) (width 0.5) (layer F.Cu) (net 9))
 (segment (start 173.495 94.195) (end 177.835 98.535) (width 0.5) (layer F.Cu) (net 9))
 (segment (start 170.335 94.195) (end 173.495 94.195) (width 0.5) (layer F.Cu) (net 9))
 (segment (start 154.975 103.615) (end 153.255 103.615) (width 0.5) (layer F.Cu) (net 18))
 (segment (start 153.255 103.615) (end 151.835 102.195) (width 0.5) (layer F.Cu) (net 18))
 (segment (start 151.835 100.36) (end 149.67 98.195) (width 0.5) (layer F.Cu) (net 18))
 (segment (start 151.835 102.195) (end 151.835 100.36) (width 0.5) (layer F.Cu) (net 18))
 (segment (start 120.385 91.195) (end 120.46 91.12) (width 0.5) (layer F.Cu) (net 2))
 (segment (start 110.835 91.195) (end 120.385 91.195) (width 0.5) (layer F.Cu) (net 2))
 (segment (start 118.835 116.695) (end 131.835 116.695) (width 0.5) (layer F.Cu) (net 25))
 (segment (start 131.835 116.695) (end 145.335 116.695) (width 0.5) (layer F.Cu) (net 25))
 (segment (start 145.335 116.695) (end 146.835 116.695) (width 0.5) (layer F.Cu) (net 25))
 (segment (start 149.67 113.86) (end 149.67 108.355) (width 0.5) (layer F.Cu) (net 25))
 (segment (start 146.835 116.695) (end 149.67 113.86) (width 0.5) (layer F.Cu) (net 25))
 (segment (start 110.735 100.195) (end 110.735 96.795) (width 0.5) (layer F.Cu) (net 21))
 (segment (start 110.735 96.795) (end 114.335 93.195) (width 0.5) (layer F.Cu) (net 21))
 (segment (start 127.91 93.195) (end 129.985 91.12) (width 0.5) (layer F.Cu) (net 21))
 (segment (start 114.335 93.195) (end 127.91 93.195) (width 0.5) (layer F.Cu) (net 21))
 (segment (start 110.735 108.595) (end 113.335 111.195) (width 0.5) (layer F.Cu) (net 21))
 (segment (start 110.735 100.195) (end 110.735 108.595) (width 0.5) (layer F.Cu) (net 21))
 (segment (start 110.835 88.695) (end 109.835 88.695) (width 0.5) (layer F.Cu) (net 1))
 (segment (start 108.735 89.795) (end 108.735 100.195) (width 0.5) (layer F.Cu) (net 1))
 (segment (start 109.835 88.695) (end 108.735 89.795) (width 0.5) (layer F.Cu) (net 1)))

